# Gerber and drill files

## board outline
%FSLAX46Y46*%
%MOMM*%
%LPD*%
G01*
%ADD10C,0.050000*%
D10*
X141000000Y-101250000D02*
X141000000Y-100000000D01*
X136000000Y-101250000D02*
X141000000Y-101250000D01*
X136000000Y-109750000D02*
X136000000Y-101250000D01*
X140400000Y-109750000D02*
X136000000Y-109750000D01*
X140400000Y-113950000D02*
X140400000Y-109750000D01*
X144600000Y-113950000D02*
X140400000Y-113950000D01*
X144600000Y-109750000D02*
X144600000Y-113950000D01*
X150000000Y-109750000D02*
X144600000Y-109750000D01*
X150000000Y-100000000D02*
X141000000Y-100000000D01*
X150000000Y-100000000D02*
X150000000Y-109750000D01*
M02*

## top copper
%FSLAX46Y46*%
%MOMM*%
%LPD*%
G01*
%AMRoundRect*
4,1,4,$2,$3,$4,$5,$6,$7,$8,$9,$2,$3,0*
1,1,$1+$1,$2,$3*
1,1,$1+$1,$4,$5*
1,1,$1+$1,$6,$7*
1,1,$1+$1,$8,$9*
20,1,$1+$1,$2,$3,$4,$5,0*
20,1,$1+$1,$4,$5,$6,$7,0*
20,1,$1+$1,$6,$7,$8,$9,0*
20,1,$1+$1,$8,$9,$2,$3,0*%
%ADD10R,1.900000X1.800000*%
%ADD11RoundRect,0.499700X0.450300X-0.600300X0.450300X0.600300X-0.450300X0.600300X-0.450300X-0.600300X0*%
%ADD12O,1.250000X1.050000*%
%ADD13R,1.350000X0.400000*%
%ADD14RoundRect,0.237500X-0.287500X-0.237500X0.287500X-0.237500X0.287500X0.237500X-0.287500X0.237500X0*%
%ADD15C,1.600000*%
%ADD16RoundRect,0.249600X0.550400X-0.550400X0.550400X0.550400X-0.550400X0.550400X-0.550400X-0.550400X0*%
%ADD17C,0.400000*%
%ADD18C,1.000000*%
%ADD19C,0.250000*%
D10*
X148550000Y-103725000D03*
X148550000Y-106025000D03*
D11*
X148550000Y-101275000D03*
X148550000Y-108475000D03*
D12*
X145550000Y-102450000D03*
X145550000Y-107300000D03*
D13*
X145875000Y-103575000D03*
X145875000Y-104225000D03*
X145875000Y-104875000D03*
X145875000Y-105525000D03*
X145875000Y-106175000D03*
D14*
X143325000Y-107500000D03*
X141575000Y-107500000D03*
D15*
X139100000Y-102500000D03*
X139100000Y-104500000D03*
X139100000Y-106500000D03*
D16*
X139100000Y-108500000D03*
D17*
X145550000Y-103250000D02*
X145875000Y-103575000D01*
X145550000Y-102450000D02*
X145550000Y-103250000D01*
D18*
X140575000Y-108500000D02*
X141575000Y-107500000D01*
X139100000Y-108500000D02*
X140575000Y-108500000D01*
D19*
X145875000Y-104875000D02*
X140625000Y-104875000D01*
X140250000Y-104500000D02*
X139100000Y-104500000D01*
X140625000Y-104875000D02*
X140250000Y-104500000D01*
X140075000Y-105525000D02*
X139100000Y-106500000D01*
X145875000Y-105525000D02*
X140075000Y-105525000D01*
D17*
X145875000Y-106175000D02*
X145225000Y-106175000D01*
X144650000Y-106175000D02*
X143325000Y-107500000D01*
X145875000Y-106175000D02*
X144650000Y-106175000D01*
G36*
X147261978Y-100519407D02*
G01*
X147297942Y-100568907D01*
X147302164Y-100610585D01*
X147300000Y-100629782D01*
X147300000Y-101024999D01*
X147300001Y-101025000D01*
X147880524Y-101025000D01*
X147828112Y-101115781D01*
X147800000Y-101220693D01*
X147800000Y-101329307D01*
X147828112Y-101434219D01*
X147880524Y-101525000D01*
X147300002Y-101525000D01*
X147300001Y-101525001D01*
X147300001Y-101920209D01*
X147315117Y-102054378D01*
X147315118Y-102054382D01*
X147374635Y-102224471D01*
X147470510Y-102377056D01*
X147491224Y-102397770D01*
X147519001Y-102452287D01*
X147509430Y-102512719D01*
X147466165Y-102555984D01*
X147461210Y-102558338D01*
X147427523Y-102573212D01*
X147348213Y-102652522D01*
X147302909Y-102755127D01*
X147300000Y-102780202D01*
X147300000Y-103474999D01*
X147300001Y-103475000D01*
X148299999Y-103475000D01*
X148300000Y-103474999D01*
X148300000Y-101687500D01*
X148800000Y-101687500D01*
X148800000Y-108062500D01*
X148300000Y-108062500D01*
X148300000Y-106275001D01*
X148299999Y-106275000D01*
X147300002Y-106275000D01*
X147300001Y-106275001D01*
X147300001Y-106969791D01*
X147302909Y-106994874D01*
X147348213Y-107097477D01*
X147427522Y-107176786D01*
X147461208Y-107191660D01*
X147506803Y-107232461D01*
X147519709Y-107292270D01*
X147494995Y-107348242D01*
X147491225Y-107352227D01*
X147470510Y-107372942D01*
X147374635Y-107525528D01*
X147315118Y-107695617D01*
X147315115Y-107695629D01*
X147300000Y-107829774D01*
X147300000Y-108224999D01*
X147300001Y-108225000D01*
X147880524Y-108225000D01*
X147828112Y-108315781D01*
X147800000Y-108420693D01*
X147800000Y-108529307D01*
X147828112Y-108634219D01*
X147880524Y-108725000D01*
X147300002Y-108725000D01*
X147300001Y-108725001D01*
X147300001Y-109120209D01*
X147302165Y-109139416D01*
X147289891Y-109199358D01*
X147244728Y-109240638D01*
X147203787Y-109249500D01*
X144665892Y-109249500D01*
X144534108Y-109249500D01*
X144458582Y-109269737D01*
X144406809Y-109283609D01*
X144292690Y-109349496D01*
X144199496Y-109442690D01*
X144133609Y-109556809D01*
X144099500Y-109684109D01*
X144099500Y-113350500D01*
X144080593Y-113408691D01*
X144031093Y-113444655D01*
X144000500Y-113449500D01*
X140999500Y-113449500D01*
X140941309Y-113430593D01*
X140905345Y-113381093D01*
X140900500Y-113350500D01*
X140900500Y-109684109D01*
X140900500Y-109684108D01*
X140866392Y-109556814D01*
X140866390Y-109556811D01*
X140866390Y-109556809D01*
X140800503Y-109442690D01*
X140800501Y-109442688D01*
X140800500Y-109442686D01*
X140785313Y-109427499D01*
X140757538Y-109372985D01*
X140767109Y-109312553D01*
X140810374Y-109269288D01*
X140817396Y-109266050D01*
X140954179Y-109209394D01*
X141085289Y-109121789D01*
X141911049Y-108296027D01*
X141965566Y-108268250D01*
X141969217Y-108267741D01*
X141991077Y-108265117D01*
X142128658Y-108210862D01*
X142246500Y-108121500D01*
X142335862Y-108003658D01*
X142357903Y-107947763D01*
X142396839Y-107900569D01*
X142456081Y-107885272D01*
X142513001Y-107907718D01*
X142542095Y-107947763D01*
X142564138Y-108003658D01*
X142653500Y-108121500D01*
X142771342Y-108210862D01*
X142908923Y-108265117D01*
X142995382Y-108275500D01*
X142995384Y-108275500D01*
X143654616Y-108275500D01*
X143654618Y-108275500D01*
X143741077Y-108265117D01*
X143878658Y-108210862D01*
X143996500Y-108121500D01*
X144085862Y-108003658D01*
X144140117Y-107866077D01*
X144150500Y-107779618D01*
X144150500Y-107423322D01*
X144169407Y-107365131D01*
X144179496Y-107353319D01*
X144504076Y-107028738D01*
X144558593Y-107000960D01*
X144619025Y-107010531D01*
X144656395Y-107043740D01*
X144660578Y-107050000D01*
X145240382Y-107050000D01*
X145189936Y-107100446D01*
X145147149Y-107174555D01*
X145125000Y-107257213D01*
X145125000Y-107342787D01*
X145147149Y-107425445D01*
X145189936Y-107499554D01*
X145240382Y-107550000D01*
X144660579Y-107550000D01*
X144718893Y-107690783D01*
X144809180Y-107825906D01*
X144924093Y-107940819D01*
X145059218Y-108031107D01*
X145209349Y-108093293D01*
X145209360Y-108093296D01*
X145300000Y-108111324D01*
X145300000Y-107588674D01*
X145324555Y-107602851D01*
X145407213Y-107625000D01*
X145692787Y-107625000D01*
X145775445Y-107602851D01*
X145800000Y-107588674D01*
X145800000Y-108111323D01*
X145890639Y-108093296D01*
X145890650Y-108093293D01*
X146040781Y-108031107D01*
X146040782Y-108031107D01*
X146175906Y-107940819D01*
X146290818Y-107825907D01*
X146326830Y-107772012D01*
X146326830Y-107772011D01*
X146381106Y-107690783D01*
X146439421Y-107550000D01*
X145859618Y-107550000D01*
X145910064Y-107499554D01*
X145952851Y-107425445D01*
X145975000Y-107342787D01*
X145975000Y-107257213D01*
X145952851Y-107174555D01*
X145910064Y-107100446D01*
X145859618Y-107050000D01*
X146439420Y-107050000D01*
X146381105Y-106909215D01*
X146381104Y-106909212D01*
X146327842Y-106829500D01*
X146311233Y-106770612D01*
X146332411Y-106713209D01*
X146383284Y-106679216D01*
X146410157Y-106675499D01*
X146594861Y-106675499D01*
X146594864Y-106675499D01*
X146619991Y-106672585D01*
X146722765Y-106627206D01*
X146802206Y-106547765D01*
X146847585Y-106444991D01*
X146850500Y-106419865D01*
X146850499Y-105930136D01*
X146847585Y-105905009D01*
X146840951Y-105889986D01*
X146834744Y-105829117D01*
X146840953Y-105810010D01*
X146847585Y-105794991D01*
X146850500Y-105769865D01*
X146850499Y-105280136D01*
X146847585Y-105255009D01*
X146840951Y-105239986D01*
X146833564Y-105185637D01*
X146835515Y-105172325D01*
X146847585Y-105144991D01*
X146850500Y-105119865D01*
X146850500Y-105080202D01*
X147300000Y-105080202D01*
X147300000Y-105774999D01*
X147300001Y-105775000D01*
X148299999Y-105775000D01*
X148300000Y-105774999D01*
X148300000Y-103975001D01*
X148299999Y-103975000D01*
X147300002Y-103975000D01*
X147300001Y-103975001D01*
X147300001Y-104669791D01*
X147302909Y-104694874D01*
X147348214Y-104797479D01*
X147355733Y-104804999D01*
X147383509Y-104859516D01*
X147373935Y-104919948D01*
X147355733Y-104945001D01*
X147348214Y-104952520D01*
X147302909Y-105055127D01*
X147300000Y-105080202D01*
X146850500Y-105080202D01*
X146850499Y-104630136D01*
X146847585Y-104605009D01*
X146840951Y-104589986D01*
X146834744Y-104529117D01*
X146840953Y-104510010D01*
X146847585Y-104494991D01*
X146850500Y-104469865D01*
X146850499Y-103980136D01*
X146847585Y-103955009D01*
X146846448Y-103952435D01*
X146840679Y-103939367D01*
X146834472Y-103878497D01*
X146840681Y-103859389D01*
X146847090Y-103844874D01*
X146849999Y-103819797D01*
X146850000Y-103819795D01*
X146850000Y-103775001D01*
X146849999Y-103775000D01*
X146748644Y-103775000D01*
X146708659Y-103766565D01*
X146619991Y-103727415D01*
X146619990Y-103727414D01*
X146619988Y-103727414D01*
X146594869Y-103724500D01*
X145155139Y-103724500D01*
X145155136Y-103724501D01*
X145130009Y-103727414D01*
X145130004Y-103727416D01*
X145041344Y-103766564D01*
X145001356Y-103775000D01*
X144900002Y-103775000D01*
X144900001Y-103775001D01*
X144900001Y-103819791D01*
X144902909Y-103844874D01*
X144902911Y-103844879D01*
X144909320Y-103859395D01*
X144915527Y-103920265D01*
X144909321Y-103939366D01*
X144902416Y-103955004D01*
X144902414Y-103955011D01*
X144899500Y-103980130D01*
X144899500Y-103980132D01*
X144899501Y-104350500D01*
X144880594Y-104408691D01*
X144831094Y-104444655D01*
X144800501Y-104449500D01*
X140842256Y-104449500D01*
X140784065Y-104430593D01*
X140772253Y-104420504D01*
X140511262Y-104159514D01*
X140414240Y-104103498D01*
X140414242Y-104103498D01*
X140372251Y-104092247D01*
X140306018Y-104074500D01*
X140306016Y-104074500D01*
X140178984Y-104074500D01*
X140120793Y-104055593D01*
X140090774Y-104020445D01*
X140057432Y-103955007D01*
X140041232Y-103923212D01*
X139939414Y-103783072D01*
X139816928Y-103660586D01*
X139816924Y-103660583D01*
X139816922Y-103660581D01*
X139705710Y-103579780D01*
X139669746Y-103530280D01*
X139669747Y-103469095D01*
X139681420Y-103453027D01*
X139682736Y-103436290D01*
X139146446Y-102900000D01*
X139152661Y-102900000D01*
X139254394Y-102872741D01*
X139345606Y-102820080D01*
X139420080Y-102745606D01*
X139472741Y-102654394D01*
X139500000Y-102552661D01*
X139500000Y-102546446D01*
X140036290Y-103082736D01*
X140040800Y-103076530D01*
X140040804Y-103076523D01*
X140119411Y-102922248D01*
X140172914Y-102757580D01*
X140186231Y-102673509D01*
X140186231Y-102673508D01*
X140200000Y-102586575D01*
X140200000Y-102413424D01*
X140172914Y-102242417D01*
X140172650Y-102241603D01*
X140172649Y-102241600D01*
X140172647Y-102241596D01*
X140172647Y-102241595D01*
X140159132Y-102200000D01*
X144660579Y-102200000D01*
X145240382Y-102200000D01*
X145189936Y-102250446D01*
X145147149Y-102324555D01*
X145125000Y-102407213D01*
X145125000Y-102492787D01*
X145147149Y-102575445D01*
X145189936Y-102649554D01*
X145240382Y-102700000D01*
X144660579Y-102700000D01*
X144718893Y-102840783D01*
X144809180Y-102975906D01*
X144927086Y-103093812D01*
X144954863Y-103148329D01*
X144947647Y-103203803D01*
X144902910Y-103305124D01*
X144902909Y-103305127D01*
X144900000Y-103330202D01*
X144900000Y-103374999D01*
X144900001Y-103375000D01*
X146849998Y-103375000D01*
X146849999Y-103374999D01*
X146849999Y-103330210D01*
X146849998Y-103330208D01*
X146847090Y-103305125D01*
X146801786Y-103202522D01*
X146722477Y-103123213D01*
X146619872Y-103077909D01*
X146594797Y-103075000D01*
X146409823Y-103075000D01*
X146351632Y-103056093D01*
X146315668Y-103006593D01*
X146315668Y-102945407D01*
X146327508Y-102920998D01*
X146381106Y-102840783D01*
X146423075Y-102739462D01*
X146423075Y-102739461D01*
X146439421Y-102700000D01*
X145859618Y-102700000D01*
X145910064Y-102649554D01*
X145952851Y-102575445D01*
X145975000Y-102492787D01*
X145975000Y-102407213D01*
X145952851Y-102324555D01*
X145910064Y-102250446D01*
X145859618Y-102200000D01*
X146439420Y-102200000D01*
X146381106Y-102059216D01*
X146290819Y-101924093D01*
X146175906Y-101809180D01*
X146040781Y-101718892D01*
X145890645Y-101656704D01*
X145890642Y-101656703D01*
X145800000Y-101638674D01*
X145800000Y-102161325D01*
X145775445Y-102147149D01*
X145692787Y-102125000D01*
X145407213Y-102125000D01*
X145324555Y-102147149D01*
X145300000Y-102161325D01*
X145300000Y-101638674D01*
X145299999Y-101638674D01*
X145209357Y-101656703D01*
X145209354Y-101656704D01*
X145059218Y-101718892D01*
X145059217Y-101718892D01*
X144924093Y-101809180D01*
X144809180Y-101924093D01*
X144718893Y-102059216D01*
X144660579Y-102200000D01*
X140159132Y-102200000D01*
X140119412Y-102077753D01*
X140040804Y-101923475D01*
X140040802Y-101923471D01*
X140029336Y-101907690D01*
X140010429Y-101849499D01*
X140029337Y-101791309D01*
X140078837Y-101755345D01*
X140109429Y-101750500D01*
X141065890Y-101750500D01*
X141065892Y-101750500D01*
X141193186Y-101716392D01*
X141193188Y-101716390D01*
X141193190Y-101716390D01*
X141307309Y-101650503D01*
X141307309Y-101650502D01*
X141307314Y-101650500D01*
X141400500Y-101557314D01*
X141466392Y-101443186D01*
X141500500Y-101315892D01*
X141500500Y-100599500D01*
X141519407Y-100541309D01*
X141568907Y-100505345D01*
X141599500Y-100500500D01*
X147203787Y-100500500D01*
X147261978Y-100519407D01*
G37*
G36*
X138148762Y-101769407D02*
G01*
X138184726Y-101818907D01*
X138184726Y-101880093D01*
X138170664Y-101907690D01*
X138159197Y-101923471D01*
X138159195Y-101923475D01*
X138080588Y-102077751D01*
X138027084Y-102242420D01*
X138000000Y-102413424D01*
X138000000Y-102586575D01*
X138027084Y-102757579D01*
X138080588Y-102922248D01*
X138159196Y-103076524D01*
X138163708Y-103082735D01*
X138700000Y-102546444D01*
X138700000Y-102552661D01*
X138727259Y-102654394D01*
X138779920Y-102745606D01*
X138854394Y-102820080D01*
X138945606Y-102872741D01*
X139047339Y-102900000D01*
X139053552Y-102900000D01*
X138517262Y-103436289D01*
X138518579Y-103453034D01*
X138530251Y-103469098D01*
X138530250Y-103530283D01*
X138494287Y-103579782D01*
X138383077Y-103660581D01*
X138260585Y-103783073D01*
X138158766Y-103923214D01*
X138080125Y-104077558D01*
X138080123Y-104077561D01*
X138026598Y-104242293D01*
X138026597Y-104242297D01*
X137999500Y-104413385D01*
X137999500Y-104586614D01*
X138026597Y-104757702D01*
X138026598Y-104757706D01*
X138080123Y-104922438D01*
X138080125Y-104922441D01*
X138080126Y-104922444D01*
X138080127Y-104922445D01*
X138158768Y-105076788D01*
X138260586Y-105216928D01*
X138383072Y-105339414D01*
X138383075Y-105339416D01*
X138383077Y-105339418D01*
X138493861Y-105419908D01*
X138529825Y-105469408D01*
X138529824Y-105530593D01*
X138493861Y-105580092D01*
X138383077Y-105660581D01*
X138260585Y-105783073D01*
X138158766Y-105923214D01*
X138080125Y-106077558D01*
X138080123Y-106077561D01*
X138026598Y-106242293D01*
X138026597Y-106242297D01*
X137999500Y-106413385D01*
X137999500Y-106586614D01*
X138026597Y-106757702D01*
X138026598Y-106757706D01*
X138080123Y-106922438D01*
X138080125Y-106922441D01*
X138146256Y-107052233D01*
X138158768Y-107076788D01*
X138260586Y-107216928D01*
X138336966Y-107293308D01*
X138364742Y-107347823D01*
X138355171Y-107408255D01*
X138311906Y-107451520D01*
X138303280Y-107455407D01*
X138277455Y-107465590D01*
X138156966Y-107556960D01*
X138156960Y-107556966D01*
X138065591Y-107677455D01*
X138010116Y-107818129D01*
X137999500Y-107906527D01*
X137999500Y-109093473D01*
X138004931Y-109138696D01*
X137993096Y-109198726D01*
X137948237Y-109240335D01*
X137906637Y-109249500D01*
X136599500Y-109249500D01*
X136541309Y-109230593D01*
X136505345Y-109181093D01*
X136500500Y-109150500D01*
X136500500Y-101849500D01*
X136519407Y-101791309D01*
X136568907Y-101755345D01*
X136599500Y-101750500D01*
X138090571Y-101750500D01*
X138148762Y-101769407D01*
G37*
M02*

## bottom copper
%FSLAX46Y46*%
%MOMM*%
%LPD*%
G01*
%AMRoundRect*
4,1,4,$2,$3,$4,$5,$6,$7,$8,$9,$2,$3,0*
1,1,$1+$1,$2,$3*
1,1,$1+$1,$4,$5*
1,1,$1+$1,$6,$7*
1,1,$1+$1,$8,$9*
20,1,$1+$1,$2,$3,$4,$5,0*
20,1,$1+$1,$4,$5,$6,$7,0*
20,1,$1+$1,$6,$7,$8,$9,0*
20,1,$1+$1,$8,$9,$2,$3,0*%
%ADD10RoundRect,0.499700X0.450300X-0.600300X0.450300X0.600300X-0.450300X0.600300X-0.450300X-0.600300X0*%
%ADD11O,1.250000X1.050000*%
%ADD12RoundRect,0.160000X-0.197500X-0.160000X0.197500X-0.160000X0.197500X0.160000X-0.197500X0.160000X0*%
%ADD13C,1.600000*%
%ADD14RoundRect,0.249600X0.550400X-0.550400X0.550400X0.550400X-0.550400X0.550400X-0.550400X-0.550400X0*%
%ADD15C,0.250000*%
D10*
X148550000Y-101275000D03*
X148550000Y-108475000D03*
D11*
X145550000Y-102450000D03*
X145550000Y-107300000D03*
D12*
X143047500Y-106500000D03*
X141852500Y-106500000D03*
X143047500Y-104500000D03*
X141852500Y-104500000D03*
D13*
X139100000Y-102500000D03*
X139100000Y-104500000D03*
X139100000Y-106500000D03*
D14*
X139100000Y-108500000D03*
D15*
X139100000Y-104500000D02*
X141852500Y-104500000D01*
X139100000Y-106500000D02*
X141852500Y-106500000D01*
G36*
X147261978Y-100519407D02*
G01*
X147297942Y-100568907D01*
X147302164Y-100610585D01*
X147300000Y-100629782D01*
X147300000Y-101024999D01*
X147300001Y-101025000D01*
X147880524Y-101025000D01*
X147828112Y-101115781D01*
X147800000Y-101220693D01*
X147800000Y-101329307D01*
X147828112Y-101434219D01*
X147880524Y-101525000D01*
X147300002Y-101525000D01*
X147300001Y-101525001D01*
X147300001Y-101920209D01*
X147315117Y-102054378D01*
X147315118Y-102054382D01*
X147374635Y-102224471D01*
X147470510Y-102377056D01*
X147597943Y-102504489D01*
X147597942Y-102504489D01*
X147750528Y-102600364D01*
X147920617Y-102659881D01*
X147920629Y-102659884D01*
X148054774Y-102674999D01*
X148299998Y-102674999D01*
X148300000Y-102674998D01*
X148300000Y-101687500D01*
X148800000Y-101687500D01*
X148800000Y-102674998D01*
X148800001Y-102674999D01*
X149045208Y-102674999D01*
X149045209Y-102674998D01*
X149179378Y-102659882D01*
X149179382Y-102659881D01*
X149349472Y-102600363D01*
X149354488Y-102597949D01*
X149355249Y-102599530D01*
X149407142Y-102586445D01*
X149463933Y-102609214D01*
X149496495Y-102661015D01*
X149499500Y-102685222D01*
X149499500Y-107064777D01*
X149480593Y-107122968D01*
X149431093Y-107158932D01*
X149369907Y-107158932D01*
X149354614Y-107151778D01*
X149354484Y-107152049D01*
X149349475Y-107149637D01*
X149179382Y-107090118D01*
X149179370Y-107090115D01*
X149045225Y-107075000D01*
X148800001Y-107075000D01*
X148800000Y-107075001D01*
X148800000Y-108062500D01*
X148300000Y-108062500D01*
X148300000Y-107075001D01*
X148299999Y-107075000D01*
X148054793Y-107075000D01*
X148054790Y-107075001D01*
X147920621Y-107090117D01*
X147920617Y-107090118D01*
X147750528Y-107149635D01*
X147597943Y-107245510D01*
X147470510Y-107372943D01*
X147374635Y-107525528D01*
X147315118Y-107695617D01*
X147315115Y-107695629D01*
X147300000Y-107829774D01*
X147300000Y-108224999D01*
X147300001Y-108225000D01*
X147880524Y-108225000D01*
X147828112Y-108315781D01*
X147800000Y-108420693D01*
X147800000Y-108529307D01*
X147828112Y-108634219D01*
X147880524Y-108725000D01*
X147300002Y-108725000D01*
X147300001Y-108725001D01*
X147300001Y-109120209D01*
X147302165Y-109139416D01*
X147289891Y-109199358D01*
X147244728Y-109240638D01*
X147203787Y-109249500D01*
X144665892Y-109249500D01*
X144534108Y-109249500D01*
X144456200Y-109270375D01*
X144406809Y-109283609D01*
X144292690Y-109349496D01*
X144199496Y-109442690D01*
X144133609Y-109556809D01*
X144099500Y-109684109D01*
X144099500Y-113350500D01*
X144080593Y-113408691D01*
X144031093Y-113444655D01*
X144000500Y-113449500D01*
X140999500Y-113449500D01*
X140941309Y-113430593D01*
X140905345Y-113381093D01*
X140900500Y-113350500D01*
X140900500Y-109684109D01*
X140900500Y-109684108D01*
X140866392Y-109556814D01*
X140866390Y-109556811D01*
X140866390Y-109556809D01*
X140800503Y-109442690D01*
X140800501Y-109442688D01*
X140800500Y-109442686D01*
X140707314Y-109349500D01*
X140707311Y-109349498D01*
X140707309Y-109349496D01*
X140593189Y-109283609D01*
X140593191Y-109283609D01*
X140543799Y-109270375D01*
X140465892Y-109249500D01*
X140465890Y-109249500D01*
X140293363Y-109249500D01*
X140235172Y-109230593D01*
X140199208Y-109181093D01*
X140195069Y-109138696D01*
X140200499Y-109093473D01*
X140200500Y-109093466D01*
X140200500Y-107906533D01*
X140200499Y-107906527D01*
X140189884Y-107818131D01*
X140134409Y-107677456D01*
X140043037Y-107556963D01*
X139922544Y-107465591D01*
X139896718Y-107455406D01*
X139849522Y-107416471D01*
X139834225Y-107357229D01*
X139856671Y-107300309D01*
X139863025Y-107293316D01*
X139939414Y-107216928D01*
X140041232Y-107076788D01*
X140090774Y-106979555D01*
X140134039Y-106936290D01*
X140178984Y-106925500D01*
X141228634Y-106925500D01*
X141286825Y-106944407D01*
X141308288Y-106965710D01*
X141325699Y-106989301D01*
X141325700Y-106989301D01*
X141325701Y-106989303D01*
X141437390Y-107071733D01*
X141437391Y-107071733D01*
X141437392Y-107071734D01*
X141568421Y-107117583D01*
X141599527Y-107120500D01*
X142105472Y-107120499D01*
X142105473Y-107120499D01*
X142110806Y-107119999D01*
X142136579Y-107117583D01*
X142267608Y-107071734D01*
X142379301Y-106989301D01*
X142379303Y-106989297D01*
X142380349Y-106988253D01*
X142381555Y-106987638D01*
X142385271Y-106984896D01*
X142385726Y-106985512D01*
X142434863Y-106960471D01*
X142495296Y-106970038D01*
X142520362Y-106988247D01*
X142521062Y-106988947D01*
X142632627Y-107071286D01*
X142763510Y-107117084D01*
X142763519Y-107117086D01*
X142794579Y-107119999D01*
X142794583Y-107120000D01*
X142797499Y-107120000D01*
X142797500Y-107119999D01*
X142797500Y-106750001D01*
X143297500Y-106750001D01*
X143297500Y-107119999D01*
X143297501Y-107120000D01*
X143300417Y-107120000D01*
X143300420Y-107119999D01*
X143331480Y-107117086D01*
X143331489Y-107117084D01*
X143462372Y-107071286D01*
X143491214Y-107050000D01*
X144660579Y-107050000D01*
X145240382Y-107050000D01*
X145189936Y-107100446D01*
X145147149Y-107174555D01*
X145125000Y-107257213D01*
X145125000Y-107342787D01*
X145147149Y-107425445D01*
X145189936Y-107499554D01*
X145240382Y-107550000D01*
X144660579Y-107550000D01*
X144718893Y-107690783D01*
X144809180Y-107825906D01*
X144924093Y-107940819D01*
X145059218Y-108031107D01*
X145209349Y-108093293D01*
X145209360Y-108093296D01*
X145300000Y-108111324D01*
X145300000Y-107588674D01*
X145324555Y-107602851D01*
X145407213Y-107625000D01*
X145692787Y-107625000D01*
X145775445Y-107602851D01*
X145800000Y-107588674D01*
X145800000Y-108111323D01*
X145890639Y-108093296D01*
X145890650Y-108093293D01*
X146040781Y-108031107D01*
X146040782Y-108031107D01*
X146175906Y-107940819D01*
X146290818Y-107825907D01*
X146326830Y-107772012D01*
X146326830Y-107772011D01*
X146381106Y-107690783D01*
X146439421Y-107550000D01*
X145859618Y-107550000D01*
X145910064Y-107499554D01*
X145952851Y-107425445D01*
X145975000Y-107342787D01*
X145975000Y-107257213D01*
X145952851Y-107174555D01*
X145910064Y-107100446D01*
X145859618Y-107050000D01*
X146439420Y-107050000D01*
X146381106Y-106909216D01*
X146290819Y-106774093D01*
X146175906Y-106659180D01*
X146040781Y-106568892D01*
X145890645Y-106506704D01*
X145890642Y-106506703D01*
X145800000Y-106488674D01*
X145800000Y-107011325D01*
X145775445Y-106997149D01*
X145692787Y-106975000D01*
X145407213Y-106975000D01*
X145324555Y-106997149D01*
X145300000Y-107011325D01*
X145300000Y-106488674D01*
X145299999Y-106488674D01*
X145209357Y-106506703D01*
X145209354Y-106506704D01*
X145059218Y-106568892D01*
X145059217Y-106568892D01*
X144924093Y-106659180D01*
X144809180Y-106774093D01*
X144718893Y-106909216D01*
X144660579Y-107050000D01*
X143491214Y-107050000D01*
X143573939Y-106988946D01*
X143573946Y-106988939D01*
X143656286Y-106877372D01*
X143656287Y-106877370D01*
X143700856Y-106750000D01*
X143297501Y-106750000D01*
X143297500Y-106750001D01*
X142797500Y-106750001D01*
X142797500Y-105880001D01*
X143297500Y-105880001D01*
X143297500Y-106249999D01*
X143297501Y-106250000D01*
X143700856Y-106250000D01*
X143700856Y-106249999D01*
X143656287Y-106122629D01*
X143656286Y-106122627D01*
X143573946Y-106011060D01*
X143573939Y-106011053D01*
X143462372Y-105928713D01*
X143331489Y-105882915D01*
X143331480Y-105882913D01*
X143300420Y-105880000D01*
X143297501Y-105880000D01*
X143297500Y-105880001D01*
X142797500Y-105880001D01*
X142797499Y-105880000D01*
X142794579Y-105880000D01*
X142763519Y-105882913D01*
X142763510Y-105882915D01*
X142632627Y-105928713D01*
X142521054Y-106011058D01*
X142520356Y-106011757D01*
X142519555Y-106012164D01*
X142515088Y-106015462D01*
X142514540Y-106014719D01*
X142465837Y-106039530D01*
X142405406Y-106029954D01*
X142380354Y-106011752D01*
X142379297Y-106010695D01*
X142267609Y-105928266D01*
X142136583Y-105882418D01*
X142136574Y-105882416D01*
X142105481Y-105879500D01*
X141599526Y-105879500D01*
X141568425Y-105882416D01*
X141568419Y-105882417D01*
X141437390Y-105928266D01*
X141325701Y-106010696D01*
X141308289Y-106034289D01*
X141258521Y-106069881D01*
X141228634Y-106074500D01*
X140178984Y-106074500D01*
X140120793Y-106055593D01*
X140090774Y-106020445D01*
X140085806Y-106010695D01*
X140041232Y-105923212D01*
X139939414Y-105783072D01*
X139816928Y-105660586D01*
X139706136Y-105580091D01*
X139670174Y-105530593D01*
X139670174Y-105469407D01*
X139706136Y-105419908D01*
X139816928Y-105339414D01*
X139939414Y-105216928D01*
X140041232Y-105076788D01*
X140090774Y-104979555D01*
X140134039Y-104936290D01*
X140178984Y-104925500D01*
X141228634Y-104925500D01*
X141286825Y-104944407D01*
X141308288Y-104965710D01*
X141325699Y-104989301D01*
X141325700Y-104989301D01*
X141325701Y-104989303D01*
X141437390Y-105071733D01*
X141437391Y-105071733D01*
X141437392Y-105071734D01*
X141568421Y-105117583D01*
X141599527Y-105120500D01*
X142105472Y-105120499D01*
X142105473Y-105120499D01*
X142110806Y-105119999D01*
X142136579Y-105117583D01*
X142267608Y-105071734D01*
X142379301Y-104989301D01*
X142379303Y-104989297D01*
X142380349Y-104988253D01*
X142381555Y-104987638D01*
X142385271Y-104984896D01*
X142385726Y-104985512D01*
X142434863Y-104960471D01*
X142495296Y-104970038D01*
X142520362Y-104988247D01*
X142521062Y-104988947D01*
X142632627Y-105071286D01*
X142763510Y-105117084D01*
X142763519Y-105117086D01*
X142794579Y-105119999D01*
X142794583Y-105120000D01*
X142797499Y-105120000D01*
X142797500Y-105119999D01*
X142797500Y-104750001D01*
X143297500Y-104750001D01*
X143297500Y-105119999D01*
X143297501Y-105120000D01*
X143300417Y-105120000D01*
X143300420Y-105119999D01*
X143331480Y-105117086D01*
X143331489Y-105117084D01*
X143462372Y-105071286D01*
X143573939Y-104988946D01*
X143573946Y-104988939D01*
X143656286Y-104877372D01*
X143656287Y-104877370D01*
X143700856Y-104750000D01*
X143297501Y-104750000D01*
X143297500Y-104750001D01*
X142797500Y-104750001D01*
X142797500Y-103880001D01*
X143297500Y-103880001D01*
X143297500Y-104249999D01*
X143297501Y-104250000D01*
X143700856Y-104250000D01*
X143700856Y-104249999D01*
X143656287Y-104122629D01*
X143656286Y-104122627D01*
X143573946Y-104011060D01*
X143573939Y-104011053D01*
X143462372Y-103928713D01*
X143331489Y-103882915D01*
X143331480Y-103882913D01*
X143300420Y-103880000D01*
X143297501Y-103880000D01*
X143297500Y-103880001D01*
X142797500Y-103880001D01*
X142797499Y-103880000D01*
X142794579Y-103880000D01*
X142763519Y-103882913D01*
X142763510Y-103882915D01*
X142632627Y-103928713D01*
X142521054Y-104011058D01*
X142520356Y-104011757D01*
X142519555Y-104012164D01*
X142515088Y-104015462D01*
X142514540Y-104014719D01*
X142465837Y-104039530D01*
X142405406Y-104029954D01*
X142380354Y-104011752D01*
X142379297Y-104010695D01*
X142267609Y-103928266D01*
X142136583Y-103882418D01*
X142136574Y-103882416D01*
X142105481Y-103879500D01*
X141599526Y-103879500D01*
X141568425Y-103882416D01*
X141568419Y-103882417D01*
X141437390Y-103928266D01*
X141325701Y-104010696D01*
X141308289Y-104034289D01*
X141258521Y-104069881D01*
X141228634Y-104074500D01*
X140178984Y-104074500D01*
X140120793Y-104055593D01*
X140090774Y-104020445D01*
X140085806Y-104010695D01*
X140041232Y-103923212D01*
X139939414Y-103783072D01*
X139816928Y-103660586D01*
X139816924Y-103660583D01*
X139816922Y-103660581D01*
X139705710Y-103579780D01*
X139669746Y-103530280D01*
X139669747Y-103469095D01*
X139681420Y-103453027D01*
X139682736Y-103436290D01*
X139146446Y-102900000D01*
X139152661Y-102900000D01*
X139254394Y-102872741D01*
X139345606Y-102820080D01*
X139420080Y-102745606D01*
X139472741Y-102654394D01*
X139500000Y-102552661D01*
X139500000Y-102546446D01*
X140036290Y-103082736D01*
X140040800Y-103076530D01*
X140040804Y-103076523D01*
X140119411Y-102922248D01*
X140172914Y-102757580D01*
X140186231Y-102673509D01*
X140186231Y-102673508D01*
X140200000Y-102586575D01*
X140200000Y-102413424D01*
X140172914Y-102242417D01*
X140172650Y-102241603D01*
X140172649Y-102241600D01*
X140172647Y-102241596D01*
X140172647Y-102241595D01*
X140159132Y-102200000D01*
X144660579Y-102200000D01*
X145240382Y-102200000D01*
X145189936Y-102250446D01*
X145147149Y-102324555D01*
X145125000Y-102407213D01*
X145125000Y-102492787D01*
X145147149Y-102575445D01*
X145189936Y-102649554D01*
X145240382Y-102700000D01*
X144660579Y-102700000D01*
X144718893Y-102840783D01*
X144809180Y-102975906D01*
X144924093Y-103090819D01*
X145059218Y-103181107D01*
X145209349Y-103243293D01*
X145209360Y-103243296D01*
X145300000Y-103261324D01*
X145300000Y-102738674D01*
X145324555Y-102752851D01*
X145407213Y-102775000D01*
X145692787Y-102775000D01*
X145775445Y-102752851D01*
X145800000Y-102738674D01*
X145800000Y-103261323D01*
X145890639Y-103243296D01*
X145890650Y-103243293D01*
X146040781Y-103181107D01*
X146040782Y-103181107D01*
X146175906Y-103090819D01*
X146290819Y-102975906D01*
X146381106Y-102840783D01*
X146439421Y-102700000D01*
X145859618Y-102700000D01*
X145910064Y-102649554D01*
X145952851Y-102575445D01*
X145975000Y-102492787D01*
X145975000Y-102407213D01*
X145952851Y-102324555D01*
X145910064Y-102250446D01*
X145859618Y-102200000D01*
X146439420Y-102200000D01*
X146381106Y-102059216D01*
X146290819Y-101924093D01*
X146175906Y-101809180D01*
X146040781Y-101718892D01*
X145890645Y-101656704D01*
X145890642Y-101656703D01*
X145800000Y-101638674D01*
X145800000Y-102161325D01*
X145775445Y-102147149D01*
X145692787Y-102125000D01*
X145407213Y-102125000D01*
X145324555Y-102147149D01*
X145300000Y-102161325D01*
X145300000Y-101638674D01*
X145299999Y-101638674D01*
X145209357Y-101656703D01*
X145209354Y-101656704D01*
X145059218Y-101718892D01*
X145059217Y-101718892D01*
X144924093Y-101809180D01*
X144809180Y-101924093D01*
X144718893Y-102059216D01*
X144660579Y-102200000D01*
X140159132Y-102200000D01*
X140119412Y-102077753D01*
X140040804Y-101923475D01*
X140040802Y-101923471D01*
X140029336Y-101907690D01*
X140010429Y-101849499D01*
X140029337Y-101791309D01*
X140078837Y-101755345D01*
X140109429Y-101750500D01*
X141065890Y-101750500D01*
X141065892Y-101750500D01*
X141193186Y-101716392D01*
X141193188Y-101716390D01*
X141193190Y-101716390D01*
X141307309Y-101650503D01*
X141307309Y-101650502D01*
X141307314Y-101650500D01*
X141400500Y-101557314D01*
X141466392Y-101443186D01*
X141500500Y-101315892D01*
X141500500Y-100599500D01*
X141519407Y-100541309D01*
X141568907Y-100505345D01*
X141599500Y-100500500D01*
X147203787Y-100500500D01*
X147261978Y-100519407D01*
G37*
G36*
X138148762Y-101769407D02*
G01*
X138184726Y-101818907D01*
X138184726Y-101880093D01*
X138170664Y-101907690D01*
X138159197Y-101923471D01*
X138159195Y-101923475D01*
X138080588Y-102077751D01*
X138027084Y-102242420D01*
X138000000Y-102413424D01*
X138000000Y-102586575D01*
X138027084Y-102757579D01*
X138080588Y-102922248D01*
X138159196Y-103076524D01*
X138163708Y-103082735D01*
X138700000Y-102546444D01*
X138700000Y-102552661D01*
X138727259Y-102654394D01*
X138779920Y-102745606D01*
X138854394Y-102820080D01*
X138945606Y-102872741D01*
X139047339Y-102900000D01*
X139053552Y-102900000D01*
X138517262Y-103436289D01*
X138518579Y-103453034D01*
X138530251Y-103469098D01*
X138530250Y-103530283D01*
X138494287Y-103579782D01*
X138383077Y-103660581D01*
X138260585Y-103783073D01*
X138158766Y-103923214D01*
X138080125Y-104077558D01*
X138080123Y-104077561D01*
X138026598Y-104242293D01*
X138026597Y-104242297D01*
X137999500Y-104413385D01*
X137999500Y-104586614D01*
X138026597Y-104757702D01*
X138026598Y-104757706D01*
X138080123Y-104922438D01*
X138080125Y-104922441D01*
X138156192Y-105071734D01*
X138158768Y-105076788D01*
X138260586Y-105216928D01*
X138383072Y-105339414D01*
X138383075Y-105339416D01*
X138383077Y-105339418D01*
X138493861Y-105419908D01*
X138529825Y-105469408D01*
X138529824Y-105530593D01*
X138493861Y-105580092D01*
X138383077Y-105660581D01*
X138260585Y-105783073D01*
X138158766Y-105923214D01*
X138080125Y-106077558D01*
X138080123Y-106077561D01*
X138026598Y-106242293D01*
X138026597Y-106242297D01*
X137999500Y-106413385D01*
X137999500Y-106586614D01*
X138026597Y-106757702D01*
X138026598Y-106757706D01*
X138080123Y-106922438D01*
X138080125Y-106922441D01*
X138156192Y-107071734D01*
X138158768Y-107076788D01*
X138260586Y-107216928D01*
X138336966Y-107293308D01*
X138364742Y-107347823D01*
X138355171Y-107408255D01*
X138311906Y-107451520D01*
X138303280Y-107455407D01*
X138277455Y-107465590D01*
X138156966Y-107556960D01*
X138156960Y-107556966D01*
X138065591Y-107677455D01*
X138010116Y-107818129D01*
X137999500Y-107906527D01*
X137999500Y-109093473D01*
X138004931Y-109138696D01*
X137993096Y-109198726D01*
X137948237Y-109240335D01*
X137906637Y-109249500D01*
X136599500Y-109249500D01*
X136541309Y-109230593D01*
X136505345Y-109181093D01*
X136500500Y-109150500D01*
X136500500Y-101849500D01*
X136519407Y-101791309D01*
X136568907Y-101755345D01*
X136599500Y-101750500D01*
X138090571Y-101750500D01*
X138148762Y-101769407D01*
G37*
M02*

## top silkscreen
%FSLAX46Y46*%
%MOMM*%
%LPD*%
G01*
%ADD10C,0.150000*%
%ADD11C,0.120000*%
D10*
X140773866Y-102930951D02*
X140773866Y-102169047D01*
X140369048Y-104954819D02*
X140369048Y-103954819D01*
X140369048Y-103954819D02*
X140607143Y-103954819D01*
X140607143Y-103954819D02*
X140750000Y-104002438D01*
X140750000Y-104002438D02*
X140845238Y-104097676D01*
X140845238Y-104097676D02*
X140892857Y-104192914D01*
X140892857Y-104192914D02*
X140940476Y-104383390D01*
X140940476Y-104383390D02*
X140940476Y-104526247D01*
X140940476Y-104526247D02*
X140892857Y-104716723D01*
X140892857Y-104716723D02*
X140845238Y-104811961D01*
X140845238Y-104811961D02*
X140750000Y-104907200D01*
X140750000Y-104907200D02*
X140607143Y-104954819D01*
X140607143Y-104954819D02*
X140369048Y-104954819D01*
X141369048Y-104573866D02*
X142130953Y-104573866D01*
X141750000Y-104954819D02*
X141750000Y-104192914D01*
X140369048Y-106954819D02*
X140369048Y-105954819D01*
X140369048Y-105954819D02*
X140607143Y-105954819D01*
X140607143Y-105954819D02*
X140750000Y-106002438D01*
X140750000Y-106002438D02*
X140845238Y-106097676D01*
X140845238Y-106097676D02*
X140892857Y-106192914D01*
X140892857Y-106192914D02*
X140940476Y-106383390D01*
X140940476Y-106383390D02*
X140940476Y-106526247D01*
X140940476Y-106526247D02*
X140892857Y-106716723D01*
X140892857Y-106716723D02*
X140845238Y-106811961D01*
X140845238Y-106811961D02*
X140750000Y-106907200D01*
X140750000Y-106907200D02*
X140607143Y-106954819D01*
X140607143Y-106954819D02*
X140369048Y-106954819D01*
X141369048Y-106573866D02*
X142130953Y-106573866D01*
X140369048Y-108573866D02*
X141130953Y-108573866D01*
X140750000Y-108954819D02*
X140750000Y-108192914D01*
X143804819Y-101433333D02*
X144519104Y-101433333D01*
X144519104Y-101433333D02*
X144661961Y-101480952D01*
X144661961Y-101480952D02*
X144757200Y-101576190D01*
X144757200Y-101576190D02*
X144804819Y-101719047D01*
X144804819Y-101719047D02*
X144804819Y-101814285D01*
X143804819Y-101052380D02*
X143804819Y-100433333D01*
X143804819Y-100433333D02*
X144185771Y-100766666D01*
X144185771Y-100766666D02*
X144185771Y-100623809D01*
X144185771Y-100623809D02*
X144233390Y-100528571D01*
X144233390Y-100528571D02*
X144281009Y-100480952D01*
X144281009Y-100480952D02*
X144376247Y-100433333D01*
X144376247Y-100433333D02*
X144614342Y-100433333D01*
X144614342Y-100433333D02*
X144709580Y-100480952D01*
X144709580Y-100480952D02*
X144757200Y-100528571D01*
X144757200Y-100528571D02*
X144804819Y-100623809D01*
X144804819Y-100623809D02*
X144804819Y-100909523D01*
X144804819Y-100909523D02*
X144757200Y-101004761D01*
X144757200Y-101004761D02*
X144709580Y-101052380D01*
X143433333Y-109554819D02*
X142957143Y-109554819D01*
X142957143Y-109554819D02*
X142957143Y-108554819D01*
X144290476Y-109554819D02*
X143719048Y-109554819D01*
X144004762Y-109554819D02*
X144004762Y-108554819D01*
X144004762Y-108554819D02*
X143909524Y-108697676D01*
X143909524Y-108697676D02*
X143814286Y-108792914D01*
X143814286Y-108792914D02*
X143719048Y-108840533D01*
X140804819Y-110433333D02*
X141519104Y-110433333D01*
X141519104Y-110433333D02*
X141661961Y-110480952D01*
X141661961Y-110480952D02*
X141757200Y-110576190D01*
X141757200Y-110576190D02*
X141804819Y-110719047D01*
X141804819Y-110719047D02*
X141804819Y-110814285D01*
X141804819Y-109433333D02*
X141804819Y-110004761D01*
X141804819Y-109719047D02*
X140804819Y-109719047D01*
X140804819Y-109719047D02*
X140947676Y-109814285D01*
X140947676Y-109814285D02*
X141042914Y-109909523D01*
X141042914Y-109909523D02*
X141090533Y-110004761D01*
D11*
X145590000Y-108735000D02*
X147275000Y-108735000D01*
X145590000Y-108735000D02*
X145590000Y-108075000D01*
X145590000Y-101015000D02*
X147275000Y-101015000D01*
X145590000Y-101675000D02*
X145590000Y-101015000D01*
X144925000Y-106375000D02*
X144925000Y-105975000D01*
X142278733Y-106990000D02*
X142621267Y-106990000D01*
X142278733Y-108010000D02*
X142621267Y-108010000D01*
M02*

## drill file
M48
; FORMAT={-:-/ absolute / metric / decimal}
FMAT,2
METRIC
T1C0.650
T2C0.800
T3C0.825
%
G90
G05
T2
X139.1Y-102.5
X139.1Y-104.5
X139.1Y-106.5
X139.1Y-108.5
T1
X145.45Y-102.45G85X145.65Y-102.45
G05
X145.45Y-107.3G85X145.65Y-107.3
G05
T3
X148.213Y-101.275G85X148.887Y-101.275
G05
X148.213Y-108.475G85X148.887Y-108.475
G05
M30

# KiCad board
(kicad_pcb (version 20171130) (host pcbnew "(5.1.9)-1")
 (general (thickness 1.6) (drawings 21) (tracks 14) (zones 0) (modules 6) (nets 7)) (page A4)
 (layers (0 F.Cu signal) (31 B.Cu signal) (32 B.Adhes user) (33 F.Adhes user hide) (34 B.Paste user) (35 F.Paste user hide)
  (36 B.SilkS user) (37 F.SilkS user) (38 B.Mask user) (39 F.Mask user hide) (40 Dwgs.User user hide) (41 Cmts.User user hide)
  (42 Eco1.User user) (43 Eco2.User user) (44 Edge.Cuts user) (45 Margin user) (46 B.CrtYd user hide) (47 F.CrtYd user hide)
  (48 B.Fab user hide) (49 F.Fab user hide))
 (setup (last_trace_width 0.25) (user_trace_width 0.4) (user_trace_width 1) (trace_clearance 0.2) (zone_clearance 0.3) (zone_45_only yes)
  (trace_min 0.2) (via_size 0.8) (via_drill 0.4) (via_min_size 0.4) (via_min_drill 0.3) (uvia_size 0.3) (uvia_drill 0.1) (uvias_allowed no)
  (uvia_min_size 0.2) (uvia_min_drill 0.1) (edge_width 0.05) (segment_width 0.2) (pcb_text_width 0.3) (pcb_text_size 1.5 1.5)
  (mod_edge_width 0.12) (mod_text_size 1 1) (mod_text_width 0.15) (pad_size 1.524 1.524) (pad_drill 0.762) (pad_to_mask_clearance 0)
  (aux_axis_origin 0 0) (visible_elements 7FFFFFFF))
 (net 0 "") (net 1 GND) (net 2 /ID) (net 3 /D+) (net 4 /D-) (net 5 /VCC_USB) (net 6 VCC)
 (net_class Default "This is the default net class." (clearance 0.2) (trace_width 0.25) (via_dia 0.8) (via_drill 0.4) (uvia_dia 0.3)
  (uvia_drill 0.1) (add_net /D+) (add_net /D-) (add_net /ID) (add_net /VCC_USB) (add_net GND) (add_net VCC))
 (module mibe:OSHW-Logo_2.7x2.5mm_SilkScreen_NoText (layer B.Cu) (at 142.5 111.85 180)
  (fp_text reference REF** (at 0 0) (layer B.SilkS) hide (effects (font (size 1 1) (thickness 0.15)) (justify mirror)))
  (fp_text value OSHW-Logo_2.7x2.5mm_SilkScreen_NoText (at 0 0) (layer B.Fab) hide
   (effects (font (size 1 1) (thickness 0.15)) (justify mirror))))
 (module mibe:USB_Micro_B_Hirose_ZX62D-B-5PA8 (layer F.Cu) (at 145.875 104.875 90)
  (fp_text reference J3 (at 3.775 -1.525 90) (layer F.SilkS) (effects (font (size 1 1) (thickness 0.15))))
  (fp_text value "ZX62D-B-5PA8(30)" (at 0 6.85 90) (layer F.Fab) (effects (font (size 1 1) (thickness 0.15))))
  (fp_line (start -3.86 -0.285) (end -3.86 1.4) (layer F.SilkS) (width 0.12))
  (fp_line (start -3.86 -0.285) (end -3.2 -0.285) (layer F.SilkS) (width 0.12))
  (fp_line (start 3.86 -0.285) (end 3.86 1.4) (layer F.SilkS) (width 0.12))
  (fp_line (start 3.2 -0.285) (end 3.86 -0.285) (layer F.SilkS) (width 0.12))
  (fp_line (start -1.5 -0.95) (end -1.1 -0.95) (layer F.SilkS) (width 0.12))
  (pad 6 smd rect (at 1.15 2.675 90) (size 1.8 1.9) (layers F.Cu F.Paste F.Mask) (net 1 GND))
  (pad 6 smd rect (at -1.15 2.675 90) (size 1.8 1.9) (layers F.Cu F.Paste F.Mask) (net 1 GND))
  (pad 6 thru_hole roundrect (at 3.6 2.675 90) (size 2.2 1.9) (drill oval 0.825 1.5) (layers *.Cu *.Mask) (roundrect_rratio 0.263)
   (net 1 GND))
  (pad 6 thru_hole roundrect (at -3.6 2.675 90) (size 2.2 1.9) (drill oval 0.825 1.5) (layers *.Cu *.Mask) (roundrect_rratio 0.263)
   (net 1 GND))
  (pad 6 thru_hole oval (at 2.425 -0.325 90) (size 1.05 1.25) (drill oval 0.65 0.85) (layers *.Cu *.Mask) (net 1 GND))
  (pad 6 thru_hole oval (at -2.425 -0.325 90) (size 1.05 1.25) (drill oval 0.65 0.85) (layers *.Cu *.Mask) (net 1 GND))
  (pad 5 smd rect (at 1.3 0 90) (size 0.4 1.35) (layers F.Cu F.Paste F.Mask) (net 1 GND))
  (pad 4 smd rect (at 0.65 0 90) (size 0.4 1.35) (layers F.Cu F.Paste F.Mask) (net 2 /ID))
  (pad 3 smd rect (at 0 0 90) (size 0.4 1.35) (layers F.Cu F.Paste F.Mask) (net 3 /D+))
  (pad 2 smd rect (at -0.65 0 90) (size 0.4 1.35) (layers F.Cu F.Paste F.Mask) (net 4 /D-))
  (pad 1 smd rect (at -1.3 0 90) (size 0.4 1.35) (layers F.Cu F.Paste F.Mask) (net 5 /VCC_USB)))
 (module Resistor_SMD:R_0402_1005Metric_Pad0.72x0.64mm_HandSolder (layer B.Cu) (at 142.45 106.5)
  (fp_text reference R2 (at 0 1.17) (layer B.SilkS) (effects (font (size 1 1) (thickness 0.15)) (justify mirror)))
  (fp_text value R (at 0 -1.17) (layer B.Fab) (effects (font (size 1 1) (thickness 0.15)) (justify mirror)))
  (pad 2 smd roundrect (at 0.5975 0) (size 0.715 0.64) (layers B.Cu B.Paste B.Mask) (roundrect_rratio 0.25) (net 1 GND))
  (pad 1 smd roundrect (at -0.5975 0) (size 0.715 0.64) (layers B.Cu B.Paste B.Mask) (roundrect_rratio 0.25) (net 4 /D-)))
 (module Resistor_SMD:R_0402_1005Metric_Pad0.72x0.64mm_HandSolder (layer B.Cu) (at 142.45 104.5)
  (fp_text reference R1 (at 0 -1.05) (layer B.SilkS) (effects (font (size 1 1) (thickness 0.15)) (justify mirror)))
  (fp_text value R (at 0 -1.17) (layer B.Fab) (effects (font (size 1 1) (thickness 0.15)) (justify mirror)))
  (pad 2 smd roundrect (at 0.5975 0) (size 0.715 0.64) (layers B.Cu B.Paste B.Mask) (roundrect_rratio 0.25) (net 1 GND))
  (pad 1 smd roundrect (at -0.5975 0) (size 0.715 0.64) (layers B.Cu B.Paste B.Mask) (roundrect_rratio 0.25) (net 3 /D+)))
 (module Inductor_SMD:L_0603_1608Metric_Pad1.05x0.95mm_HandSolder (layer F.Cu) (at 142.45 107.5)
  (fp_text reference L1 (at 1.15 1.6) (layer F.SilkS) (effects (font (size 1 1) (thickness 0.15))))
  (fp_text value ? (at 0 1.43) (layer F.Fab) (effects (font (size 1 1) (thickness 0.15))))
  (fp_line (start -0.171267 -0.51) (end 0.171267 -0.51) (layer F.SilkS) (width 0.12))
  (fp_line (start -0.171267 0.51) (end 0.171267 0.51) (layer F.SilkS) (width 0.12))
  (pad 2 smd roundrect (at 0.875 0) (size 1.05 0.95) (layers F.Cu F.Paste F.Mask) (roundrect_rratio 0.25) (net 5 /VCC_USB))
  (pad 1 smd roundrect (at -0.875 0) (size 1.05 0.95) (layers F.Cu F.Paste F.Mask) (roundrect_rratio 0.25) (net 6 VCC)))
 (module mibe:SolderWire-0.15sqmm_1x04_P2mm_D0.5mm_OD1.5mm (layer F.Cu) (at 139.1 108.5 90)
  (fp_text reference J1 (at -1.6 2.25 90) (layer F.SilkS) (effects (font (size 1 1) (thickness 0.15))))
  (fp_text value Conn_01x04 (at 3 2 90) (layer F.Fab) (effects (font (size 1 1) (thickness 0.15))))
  (pad 4 thru_hole circle (at 6 0 90) (size 1.6 1.6) (drill 0.8) (layers *.Cu *.Mask) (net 1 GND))
  (pad 3 thru_hole circle (at 4 0 90) (size 1.6 1.6) (drill 0.8) (layers *.Cu *.Mask) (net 3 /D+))
  (pad 2 thru_hole circle (at 2 0 90) (size 1.6 1.6) (drill 0.8) (layers *.Cu *.Mask) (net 4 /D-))
  (pad 1 thru_hole roundrect (at 0 0 90) (size 1.6 1.6) (drill 0.8) (layers *.Cu *.Mask) (roundrect_rratio 0.156) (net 6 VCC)))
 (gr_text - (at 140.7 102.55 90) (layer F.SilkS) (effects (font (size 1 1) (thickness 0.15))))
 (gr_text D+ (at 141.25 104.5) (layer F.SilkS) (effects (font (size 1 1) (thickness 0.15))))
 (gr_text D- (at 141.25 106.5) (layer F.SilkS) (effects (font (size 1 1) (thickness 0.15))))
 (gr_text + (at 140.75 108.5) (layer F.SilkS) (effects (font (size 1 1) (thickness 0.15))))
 (gr_line (start 141 101.25) (end 141 100) (layer Edge.Cuts) (width 0.05))
 (gr_line (start 136 101.25) (end 141 101.25) (layer Edge.Cuts) (width 0.05))
 (gr_line (start 136 109.75) (end 136 101.25) (layer Edge.Cuts) (width 0.05))
 (gr_line (start 140.4 109.75) (end 136 109.75) (layer Edge.Cuts) (width 0.05))
 (gr_line (start 140.4 113.95) (end 140.4 109.75) (layer Edge.Cuts) (width 0.05))
 (gr_line (start 144.6 113.95) (end 140.4 113.95) (layer Edge.Cuts) (width 0.05))
 (gr_line (start 144.6 109.75) (end 144.6 113.95) (layer Edge.Cuts) (width 0.05))
 (gr_line (start 150 109.75) (end 144.6 109.75) (layer Edge.Cuts) (width 0.05))
 (gr_line (start 150 100) (end 141 100) (layer Edge.Cuts) (width 0.05))
 (gr_line (start 150 100) (end 150 109.75) (layer Edge.Cuts) (width 0.05))
 (segment (start 145.55 103.25) (end 145.875 103.575) (width 0.4) (layer F.Cu) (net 1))
 (segment (start 145.55 102.45) (end 145.55 103.25) (width 0.4) (layer F.Cu) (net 1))
 (segment (start 140.575 108.5) (end 141.575 107.5) (width 1) (layer F.Cu) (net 6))
 (segment (start 139.1 108.5) (end 140.575 108.5) (width 1) (layer F.Cu) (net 6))
 (segment (start 145.875 104.875) (end 140.625 104.875) (width 0.25) (layer F.Cu) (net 3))
 (segment (start 140.25 104.5) (end 139.1 104.5) (width 0.25) (layer F.Cu) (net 3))
 (segment (start 140.625 104.875) (end 140.25 104.5) (width 0.25) (layer F.Cu) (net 3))
 (segment (start 139.1 104.5) (end 141.8525 104.5) (width 0.25) (layer B.Cu) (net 3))
 (segment (start 140.075 105.525) (end 139.1 106.5) (width 0.25) (layer F.Cu) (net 4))
 (segment (start 145.875 105.525) (end 140.075 105.525) (width 0.25) (layer F.Cu) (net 4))
 (segment (start 139.1 106.5) (end 141.8525 106.5) (width 0.25) (layer B.Cu) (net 4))
 (segment (start 145.875 106.175) (end 145.225 106.175) (width 0.4) (layer F.Cu) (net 5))
 (segment (start 144.65 106.175) (end 143.325 107.5) (width 0.4) (layer F.Cu) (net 5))
 (segment (start 145.875 106.175) (end 144.65 106.175) (width 0.4) (layer F.Cu) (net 5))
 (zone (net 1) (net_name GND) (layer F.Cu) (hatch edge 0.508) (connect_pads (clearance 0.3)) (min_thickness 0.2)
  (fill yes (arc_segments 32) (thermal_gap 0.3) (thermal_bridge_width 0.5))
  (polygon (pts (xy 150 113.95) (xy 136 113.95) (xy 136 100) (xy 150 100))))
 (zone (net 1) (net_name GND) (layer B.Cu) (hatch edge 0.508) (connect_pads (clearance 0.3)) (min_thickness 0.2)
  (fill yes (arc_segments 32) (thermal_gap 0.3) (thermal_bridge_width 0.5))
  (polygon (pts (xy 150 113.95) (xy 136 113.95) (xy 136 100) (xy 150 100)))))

